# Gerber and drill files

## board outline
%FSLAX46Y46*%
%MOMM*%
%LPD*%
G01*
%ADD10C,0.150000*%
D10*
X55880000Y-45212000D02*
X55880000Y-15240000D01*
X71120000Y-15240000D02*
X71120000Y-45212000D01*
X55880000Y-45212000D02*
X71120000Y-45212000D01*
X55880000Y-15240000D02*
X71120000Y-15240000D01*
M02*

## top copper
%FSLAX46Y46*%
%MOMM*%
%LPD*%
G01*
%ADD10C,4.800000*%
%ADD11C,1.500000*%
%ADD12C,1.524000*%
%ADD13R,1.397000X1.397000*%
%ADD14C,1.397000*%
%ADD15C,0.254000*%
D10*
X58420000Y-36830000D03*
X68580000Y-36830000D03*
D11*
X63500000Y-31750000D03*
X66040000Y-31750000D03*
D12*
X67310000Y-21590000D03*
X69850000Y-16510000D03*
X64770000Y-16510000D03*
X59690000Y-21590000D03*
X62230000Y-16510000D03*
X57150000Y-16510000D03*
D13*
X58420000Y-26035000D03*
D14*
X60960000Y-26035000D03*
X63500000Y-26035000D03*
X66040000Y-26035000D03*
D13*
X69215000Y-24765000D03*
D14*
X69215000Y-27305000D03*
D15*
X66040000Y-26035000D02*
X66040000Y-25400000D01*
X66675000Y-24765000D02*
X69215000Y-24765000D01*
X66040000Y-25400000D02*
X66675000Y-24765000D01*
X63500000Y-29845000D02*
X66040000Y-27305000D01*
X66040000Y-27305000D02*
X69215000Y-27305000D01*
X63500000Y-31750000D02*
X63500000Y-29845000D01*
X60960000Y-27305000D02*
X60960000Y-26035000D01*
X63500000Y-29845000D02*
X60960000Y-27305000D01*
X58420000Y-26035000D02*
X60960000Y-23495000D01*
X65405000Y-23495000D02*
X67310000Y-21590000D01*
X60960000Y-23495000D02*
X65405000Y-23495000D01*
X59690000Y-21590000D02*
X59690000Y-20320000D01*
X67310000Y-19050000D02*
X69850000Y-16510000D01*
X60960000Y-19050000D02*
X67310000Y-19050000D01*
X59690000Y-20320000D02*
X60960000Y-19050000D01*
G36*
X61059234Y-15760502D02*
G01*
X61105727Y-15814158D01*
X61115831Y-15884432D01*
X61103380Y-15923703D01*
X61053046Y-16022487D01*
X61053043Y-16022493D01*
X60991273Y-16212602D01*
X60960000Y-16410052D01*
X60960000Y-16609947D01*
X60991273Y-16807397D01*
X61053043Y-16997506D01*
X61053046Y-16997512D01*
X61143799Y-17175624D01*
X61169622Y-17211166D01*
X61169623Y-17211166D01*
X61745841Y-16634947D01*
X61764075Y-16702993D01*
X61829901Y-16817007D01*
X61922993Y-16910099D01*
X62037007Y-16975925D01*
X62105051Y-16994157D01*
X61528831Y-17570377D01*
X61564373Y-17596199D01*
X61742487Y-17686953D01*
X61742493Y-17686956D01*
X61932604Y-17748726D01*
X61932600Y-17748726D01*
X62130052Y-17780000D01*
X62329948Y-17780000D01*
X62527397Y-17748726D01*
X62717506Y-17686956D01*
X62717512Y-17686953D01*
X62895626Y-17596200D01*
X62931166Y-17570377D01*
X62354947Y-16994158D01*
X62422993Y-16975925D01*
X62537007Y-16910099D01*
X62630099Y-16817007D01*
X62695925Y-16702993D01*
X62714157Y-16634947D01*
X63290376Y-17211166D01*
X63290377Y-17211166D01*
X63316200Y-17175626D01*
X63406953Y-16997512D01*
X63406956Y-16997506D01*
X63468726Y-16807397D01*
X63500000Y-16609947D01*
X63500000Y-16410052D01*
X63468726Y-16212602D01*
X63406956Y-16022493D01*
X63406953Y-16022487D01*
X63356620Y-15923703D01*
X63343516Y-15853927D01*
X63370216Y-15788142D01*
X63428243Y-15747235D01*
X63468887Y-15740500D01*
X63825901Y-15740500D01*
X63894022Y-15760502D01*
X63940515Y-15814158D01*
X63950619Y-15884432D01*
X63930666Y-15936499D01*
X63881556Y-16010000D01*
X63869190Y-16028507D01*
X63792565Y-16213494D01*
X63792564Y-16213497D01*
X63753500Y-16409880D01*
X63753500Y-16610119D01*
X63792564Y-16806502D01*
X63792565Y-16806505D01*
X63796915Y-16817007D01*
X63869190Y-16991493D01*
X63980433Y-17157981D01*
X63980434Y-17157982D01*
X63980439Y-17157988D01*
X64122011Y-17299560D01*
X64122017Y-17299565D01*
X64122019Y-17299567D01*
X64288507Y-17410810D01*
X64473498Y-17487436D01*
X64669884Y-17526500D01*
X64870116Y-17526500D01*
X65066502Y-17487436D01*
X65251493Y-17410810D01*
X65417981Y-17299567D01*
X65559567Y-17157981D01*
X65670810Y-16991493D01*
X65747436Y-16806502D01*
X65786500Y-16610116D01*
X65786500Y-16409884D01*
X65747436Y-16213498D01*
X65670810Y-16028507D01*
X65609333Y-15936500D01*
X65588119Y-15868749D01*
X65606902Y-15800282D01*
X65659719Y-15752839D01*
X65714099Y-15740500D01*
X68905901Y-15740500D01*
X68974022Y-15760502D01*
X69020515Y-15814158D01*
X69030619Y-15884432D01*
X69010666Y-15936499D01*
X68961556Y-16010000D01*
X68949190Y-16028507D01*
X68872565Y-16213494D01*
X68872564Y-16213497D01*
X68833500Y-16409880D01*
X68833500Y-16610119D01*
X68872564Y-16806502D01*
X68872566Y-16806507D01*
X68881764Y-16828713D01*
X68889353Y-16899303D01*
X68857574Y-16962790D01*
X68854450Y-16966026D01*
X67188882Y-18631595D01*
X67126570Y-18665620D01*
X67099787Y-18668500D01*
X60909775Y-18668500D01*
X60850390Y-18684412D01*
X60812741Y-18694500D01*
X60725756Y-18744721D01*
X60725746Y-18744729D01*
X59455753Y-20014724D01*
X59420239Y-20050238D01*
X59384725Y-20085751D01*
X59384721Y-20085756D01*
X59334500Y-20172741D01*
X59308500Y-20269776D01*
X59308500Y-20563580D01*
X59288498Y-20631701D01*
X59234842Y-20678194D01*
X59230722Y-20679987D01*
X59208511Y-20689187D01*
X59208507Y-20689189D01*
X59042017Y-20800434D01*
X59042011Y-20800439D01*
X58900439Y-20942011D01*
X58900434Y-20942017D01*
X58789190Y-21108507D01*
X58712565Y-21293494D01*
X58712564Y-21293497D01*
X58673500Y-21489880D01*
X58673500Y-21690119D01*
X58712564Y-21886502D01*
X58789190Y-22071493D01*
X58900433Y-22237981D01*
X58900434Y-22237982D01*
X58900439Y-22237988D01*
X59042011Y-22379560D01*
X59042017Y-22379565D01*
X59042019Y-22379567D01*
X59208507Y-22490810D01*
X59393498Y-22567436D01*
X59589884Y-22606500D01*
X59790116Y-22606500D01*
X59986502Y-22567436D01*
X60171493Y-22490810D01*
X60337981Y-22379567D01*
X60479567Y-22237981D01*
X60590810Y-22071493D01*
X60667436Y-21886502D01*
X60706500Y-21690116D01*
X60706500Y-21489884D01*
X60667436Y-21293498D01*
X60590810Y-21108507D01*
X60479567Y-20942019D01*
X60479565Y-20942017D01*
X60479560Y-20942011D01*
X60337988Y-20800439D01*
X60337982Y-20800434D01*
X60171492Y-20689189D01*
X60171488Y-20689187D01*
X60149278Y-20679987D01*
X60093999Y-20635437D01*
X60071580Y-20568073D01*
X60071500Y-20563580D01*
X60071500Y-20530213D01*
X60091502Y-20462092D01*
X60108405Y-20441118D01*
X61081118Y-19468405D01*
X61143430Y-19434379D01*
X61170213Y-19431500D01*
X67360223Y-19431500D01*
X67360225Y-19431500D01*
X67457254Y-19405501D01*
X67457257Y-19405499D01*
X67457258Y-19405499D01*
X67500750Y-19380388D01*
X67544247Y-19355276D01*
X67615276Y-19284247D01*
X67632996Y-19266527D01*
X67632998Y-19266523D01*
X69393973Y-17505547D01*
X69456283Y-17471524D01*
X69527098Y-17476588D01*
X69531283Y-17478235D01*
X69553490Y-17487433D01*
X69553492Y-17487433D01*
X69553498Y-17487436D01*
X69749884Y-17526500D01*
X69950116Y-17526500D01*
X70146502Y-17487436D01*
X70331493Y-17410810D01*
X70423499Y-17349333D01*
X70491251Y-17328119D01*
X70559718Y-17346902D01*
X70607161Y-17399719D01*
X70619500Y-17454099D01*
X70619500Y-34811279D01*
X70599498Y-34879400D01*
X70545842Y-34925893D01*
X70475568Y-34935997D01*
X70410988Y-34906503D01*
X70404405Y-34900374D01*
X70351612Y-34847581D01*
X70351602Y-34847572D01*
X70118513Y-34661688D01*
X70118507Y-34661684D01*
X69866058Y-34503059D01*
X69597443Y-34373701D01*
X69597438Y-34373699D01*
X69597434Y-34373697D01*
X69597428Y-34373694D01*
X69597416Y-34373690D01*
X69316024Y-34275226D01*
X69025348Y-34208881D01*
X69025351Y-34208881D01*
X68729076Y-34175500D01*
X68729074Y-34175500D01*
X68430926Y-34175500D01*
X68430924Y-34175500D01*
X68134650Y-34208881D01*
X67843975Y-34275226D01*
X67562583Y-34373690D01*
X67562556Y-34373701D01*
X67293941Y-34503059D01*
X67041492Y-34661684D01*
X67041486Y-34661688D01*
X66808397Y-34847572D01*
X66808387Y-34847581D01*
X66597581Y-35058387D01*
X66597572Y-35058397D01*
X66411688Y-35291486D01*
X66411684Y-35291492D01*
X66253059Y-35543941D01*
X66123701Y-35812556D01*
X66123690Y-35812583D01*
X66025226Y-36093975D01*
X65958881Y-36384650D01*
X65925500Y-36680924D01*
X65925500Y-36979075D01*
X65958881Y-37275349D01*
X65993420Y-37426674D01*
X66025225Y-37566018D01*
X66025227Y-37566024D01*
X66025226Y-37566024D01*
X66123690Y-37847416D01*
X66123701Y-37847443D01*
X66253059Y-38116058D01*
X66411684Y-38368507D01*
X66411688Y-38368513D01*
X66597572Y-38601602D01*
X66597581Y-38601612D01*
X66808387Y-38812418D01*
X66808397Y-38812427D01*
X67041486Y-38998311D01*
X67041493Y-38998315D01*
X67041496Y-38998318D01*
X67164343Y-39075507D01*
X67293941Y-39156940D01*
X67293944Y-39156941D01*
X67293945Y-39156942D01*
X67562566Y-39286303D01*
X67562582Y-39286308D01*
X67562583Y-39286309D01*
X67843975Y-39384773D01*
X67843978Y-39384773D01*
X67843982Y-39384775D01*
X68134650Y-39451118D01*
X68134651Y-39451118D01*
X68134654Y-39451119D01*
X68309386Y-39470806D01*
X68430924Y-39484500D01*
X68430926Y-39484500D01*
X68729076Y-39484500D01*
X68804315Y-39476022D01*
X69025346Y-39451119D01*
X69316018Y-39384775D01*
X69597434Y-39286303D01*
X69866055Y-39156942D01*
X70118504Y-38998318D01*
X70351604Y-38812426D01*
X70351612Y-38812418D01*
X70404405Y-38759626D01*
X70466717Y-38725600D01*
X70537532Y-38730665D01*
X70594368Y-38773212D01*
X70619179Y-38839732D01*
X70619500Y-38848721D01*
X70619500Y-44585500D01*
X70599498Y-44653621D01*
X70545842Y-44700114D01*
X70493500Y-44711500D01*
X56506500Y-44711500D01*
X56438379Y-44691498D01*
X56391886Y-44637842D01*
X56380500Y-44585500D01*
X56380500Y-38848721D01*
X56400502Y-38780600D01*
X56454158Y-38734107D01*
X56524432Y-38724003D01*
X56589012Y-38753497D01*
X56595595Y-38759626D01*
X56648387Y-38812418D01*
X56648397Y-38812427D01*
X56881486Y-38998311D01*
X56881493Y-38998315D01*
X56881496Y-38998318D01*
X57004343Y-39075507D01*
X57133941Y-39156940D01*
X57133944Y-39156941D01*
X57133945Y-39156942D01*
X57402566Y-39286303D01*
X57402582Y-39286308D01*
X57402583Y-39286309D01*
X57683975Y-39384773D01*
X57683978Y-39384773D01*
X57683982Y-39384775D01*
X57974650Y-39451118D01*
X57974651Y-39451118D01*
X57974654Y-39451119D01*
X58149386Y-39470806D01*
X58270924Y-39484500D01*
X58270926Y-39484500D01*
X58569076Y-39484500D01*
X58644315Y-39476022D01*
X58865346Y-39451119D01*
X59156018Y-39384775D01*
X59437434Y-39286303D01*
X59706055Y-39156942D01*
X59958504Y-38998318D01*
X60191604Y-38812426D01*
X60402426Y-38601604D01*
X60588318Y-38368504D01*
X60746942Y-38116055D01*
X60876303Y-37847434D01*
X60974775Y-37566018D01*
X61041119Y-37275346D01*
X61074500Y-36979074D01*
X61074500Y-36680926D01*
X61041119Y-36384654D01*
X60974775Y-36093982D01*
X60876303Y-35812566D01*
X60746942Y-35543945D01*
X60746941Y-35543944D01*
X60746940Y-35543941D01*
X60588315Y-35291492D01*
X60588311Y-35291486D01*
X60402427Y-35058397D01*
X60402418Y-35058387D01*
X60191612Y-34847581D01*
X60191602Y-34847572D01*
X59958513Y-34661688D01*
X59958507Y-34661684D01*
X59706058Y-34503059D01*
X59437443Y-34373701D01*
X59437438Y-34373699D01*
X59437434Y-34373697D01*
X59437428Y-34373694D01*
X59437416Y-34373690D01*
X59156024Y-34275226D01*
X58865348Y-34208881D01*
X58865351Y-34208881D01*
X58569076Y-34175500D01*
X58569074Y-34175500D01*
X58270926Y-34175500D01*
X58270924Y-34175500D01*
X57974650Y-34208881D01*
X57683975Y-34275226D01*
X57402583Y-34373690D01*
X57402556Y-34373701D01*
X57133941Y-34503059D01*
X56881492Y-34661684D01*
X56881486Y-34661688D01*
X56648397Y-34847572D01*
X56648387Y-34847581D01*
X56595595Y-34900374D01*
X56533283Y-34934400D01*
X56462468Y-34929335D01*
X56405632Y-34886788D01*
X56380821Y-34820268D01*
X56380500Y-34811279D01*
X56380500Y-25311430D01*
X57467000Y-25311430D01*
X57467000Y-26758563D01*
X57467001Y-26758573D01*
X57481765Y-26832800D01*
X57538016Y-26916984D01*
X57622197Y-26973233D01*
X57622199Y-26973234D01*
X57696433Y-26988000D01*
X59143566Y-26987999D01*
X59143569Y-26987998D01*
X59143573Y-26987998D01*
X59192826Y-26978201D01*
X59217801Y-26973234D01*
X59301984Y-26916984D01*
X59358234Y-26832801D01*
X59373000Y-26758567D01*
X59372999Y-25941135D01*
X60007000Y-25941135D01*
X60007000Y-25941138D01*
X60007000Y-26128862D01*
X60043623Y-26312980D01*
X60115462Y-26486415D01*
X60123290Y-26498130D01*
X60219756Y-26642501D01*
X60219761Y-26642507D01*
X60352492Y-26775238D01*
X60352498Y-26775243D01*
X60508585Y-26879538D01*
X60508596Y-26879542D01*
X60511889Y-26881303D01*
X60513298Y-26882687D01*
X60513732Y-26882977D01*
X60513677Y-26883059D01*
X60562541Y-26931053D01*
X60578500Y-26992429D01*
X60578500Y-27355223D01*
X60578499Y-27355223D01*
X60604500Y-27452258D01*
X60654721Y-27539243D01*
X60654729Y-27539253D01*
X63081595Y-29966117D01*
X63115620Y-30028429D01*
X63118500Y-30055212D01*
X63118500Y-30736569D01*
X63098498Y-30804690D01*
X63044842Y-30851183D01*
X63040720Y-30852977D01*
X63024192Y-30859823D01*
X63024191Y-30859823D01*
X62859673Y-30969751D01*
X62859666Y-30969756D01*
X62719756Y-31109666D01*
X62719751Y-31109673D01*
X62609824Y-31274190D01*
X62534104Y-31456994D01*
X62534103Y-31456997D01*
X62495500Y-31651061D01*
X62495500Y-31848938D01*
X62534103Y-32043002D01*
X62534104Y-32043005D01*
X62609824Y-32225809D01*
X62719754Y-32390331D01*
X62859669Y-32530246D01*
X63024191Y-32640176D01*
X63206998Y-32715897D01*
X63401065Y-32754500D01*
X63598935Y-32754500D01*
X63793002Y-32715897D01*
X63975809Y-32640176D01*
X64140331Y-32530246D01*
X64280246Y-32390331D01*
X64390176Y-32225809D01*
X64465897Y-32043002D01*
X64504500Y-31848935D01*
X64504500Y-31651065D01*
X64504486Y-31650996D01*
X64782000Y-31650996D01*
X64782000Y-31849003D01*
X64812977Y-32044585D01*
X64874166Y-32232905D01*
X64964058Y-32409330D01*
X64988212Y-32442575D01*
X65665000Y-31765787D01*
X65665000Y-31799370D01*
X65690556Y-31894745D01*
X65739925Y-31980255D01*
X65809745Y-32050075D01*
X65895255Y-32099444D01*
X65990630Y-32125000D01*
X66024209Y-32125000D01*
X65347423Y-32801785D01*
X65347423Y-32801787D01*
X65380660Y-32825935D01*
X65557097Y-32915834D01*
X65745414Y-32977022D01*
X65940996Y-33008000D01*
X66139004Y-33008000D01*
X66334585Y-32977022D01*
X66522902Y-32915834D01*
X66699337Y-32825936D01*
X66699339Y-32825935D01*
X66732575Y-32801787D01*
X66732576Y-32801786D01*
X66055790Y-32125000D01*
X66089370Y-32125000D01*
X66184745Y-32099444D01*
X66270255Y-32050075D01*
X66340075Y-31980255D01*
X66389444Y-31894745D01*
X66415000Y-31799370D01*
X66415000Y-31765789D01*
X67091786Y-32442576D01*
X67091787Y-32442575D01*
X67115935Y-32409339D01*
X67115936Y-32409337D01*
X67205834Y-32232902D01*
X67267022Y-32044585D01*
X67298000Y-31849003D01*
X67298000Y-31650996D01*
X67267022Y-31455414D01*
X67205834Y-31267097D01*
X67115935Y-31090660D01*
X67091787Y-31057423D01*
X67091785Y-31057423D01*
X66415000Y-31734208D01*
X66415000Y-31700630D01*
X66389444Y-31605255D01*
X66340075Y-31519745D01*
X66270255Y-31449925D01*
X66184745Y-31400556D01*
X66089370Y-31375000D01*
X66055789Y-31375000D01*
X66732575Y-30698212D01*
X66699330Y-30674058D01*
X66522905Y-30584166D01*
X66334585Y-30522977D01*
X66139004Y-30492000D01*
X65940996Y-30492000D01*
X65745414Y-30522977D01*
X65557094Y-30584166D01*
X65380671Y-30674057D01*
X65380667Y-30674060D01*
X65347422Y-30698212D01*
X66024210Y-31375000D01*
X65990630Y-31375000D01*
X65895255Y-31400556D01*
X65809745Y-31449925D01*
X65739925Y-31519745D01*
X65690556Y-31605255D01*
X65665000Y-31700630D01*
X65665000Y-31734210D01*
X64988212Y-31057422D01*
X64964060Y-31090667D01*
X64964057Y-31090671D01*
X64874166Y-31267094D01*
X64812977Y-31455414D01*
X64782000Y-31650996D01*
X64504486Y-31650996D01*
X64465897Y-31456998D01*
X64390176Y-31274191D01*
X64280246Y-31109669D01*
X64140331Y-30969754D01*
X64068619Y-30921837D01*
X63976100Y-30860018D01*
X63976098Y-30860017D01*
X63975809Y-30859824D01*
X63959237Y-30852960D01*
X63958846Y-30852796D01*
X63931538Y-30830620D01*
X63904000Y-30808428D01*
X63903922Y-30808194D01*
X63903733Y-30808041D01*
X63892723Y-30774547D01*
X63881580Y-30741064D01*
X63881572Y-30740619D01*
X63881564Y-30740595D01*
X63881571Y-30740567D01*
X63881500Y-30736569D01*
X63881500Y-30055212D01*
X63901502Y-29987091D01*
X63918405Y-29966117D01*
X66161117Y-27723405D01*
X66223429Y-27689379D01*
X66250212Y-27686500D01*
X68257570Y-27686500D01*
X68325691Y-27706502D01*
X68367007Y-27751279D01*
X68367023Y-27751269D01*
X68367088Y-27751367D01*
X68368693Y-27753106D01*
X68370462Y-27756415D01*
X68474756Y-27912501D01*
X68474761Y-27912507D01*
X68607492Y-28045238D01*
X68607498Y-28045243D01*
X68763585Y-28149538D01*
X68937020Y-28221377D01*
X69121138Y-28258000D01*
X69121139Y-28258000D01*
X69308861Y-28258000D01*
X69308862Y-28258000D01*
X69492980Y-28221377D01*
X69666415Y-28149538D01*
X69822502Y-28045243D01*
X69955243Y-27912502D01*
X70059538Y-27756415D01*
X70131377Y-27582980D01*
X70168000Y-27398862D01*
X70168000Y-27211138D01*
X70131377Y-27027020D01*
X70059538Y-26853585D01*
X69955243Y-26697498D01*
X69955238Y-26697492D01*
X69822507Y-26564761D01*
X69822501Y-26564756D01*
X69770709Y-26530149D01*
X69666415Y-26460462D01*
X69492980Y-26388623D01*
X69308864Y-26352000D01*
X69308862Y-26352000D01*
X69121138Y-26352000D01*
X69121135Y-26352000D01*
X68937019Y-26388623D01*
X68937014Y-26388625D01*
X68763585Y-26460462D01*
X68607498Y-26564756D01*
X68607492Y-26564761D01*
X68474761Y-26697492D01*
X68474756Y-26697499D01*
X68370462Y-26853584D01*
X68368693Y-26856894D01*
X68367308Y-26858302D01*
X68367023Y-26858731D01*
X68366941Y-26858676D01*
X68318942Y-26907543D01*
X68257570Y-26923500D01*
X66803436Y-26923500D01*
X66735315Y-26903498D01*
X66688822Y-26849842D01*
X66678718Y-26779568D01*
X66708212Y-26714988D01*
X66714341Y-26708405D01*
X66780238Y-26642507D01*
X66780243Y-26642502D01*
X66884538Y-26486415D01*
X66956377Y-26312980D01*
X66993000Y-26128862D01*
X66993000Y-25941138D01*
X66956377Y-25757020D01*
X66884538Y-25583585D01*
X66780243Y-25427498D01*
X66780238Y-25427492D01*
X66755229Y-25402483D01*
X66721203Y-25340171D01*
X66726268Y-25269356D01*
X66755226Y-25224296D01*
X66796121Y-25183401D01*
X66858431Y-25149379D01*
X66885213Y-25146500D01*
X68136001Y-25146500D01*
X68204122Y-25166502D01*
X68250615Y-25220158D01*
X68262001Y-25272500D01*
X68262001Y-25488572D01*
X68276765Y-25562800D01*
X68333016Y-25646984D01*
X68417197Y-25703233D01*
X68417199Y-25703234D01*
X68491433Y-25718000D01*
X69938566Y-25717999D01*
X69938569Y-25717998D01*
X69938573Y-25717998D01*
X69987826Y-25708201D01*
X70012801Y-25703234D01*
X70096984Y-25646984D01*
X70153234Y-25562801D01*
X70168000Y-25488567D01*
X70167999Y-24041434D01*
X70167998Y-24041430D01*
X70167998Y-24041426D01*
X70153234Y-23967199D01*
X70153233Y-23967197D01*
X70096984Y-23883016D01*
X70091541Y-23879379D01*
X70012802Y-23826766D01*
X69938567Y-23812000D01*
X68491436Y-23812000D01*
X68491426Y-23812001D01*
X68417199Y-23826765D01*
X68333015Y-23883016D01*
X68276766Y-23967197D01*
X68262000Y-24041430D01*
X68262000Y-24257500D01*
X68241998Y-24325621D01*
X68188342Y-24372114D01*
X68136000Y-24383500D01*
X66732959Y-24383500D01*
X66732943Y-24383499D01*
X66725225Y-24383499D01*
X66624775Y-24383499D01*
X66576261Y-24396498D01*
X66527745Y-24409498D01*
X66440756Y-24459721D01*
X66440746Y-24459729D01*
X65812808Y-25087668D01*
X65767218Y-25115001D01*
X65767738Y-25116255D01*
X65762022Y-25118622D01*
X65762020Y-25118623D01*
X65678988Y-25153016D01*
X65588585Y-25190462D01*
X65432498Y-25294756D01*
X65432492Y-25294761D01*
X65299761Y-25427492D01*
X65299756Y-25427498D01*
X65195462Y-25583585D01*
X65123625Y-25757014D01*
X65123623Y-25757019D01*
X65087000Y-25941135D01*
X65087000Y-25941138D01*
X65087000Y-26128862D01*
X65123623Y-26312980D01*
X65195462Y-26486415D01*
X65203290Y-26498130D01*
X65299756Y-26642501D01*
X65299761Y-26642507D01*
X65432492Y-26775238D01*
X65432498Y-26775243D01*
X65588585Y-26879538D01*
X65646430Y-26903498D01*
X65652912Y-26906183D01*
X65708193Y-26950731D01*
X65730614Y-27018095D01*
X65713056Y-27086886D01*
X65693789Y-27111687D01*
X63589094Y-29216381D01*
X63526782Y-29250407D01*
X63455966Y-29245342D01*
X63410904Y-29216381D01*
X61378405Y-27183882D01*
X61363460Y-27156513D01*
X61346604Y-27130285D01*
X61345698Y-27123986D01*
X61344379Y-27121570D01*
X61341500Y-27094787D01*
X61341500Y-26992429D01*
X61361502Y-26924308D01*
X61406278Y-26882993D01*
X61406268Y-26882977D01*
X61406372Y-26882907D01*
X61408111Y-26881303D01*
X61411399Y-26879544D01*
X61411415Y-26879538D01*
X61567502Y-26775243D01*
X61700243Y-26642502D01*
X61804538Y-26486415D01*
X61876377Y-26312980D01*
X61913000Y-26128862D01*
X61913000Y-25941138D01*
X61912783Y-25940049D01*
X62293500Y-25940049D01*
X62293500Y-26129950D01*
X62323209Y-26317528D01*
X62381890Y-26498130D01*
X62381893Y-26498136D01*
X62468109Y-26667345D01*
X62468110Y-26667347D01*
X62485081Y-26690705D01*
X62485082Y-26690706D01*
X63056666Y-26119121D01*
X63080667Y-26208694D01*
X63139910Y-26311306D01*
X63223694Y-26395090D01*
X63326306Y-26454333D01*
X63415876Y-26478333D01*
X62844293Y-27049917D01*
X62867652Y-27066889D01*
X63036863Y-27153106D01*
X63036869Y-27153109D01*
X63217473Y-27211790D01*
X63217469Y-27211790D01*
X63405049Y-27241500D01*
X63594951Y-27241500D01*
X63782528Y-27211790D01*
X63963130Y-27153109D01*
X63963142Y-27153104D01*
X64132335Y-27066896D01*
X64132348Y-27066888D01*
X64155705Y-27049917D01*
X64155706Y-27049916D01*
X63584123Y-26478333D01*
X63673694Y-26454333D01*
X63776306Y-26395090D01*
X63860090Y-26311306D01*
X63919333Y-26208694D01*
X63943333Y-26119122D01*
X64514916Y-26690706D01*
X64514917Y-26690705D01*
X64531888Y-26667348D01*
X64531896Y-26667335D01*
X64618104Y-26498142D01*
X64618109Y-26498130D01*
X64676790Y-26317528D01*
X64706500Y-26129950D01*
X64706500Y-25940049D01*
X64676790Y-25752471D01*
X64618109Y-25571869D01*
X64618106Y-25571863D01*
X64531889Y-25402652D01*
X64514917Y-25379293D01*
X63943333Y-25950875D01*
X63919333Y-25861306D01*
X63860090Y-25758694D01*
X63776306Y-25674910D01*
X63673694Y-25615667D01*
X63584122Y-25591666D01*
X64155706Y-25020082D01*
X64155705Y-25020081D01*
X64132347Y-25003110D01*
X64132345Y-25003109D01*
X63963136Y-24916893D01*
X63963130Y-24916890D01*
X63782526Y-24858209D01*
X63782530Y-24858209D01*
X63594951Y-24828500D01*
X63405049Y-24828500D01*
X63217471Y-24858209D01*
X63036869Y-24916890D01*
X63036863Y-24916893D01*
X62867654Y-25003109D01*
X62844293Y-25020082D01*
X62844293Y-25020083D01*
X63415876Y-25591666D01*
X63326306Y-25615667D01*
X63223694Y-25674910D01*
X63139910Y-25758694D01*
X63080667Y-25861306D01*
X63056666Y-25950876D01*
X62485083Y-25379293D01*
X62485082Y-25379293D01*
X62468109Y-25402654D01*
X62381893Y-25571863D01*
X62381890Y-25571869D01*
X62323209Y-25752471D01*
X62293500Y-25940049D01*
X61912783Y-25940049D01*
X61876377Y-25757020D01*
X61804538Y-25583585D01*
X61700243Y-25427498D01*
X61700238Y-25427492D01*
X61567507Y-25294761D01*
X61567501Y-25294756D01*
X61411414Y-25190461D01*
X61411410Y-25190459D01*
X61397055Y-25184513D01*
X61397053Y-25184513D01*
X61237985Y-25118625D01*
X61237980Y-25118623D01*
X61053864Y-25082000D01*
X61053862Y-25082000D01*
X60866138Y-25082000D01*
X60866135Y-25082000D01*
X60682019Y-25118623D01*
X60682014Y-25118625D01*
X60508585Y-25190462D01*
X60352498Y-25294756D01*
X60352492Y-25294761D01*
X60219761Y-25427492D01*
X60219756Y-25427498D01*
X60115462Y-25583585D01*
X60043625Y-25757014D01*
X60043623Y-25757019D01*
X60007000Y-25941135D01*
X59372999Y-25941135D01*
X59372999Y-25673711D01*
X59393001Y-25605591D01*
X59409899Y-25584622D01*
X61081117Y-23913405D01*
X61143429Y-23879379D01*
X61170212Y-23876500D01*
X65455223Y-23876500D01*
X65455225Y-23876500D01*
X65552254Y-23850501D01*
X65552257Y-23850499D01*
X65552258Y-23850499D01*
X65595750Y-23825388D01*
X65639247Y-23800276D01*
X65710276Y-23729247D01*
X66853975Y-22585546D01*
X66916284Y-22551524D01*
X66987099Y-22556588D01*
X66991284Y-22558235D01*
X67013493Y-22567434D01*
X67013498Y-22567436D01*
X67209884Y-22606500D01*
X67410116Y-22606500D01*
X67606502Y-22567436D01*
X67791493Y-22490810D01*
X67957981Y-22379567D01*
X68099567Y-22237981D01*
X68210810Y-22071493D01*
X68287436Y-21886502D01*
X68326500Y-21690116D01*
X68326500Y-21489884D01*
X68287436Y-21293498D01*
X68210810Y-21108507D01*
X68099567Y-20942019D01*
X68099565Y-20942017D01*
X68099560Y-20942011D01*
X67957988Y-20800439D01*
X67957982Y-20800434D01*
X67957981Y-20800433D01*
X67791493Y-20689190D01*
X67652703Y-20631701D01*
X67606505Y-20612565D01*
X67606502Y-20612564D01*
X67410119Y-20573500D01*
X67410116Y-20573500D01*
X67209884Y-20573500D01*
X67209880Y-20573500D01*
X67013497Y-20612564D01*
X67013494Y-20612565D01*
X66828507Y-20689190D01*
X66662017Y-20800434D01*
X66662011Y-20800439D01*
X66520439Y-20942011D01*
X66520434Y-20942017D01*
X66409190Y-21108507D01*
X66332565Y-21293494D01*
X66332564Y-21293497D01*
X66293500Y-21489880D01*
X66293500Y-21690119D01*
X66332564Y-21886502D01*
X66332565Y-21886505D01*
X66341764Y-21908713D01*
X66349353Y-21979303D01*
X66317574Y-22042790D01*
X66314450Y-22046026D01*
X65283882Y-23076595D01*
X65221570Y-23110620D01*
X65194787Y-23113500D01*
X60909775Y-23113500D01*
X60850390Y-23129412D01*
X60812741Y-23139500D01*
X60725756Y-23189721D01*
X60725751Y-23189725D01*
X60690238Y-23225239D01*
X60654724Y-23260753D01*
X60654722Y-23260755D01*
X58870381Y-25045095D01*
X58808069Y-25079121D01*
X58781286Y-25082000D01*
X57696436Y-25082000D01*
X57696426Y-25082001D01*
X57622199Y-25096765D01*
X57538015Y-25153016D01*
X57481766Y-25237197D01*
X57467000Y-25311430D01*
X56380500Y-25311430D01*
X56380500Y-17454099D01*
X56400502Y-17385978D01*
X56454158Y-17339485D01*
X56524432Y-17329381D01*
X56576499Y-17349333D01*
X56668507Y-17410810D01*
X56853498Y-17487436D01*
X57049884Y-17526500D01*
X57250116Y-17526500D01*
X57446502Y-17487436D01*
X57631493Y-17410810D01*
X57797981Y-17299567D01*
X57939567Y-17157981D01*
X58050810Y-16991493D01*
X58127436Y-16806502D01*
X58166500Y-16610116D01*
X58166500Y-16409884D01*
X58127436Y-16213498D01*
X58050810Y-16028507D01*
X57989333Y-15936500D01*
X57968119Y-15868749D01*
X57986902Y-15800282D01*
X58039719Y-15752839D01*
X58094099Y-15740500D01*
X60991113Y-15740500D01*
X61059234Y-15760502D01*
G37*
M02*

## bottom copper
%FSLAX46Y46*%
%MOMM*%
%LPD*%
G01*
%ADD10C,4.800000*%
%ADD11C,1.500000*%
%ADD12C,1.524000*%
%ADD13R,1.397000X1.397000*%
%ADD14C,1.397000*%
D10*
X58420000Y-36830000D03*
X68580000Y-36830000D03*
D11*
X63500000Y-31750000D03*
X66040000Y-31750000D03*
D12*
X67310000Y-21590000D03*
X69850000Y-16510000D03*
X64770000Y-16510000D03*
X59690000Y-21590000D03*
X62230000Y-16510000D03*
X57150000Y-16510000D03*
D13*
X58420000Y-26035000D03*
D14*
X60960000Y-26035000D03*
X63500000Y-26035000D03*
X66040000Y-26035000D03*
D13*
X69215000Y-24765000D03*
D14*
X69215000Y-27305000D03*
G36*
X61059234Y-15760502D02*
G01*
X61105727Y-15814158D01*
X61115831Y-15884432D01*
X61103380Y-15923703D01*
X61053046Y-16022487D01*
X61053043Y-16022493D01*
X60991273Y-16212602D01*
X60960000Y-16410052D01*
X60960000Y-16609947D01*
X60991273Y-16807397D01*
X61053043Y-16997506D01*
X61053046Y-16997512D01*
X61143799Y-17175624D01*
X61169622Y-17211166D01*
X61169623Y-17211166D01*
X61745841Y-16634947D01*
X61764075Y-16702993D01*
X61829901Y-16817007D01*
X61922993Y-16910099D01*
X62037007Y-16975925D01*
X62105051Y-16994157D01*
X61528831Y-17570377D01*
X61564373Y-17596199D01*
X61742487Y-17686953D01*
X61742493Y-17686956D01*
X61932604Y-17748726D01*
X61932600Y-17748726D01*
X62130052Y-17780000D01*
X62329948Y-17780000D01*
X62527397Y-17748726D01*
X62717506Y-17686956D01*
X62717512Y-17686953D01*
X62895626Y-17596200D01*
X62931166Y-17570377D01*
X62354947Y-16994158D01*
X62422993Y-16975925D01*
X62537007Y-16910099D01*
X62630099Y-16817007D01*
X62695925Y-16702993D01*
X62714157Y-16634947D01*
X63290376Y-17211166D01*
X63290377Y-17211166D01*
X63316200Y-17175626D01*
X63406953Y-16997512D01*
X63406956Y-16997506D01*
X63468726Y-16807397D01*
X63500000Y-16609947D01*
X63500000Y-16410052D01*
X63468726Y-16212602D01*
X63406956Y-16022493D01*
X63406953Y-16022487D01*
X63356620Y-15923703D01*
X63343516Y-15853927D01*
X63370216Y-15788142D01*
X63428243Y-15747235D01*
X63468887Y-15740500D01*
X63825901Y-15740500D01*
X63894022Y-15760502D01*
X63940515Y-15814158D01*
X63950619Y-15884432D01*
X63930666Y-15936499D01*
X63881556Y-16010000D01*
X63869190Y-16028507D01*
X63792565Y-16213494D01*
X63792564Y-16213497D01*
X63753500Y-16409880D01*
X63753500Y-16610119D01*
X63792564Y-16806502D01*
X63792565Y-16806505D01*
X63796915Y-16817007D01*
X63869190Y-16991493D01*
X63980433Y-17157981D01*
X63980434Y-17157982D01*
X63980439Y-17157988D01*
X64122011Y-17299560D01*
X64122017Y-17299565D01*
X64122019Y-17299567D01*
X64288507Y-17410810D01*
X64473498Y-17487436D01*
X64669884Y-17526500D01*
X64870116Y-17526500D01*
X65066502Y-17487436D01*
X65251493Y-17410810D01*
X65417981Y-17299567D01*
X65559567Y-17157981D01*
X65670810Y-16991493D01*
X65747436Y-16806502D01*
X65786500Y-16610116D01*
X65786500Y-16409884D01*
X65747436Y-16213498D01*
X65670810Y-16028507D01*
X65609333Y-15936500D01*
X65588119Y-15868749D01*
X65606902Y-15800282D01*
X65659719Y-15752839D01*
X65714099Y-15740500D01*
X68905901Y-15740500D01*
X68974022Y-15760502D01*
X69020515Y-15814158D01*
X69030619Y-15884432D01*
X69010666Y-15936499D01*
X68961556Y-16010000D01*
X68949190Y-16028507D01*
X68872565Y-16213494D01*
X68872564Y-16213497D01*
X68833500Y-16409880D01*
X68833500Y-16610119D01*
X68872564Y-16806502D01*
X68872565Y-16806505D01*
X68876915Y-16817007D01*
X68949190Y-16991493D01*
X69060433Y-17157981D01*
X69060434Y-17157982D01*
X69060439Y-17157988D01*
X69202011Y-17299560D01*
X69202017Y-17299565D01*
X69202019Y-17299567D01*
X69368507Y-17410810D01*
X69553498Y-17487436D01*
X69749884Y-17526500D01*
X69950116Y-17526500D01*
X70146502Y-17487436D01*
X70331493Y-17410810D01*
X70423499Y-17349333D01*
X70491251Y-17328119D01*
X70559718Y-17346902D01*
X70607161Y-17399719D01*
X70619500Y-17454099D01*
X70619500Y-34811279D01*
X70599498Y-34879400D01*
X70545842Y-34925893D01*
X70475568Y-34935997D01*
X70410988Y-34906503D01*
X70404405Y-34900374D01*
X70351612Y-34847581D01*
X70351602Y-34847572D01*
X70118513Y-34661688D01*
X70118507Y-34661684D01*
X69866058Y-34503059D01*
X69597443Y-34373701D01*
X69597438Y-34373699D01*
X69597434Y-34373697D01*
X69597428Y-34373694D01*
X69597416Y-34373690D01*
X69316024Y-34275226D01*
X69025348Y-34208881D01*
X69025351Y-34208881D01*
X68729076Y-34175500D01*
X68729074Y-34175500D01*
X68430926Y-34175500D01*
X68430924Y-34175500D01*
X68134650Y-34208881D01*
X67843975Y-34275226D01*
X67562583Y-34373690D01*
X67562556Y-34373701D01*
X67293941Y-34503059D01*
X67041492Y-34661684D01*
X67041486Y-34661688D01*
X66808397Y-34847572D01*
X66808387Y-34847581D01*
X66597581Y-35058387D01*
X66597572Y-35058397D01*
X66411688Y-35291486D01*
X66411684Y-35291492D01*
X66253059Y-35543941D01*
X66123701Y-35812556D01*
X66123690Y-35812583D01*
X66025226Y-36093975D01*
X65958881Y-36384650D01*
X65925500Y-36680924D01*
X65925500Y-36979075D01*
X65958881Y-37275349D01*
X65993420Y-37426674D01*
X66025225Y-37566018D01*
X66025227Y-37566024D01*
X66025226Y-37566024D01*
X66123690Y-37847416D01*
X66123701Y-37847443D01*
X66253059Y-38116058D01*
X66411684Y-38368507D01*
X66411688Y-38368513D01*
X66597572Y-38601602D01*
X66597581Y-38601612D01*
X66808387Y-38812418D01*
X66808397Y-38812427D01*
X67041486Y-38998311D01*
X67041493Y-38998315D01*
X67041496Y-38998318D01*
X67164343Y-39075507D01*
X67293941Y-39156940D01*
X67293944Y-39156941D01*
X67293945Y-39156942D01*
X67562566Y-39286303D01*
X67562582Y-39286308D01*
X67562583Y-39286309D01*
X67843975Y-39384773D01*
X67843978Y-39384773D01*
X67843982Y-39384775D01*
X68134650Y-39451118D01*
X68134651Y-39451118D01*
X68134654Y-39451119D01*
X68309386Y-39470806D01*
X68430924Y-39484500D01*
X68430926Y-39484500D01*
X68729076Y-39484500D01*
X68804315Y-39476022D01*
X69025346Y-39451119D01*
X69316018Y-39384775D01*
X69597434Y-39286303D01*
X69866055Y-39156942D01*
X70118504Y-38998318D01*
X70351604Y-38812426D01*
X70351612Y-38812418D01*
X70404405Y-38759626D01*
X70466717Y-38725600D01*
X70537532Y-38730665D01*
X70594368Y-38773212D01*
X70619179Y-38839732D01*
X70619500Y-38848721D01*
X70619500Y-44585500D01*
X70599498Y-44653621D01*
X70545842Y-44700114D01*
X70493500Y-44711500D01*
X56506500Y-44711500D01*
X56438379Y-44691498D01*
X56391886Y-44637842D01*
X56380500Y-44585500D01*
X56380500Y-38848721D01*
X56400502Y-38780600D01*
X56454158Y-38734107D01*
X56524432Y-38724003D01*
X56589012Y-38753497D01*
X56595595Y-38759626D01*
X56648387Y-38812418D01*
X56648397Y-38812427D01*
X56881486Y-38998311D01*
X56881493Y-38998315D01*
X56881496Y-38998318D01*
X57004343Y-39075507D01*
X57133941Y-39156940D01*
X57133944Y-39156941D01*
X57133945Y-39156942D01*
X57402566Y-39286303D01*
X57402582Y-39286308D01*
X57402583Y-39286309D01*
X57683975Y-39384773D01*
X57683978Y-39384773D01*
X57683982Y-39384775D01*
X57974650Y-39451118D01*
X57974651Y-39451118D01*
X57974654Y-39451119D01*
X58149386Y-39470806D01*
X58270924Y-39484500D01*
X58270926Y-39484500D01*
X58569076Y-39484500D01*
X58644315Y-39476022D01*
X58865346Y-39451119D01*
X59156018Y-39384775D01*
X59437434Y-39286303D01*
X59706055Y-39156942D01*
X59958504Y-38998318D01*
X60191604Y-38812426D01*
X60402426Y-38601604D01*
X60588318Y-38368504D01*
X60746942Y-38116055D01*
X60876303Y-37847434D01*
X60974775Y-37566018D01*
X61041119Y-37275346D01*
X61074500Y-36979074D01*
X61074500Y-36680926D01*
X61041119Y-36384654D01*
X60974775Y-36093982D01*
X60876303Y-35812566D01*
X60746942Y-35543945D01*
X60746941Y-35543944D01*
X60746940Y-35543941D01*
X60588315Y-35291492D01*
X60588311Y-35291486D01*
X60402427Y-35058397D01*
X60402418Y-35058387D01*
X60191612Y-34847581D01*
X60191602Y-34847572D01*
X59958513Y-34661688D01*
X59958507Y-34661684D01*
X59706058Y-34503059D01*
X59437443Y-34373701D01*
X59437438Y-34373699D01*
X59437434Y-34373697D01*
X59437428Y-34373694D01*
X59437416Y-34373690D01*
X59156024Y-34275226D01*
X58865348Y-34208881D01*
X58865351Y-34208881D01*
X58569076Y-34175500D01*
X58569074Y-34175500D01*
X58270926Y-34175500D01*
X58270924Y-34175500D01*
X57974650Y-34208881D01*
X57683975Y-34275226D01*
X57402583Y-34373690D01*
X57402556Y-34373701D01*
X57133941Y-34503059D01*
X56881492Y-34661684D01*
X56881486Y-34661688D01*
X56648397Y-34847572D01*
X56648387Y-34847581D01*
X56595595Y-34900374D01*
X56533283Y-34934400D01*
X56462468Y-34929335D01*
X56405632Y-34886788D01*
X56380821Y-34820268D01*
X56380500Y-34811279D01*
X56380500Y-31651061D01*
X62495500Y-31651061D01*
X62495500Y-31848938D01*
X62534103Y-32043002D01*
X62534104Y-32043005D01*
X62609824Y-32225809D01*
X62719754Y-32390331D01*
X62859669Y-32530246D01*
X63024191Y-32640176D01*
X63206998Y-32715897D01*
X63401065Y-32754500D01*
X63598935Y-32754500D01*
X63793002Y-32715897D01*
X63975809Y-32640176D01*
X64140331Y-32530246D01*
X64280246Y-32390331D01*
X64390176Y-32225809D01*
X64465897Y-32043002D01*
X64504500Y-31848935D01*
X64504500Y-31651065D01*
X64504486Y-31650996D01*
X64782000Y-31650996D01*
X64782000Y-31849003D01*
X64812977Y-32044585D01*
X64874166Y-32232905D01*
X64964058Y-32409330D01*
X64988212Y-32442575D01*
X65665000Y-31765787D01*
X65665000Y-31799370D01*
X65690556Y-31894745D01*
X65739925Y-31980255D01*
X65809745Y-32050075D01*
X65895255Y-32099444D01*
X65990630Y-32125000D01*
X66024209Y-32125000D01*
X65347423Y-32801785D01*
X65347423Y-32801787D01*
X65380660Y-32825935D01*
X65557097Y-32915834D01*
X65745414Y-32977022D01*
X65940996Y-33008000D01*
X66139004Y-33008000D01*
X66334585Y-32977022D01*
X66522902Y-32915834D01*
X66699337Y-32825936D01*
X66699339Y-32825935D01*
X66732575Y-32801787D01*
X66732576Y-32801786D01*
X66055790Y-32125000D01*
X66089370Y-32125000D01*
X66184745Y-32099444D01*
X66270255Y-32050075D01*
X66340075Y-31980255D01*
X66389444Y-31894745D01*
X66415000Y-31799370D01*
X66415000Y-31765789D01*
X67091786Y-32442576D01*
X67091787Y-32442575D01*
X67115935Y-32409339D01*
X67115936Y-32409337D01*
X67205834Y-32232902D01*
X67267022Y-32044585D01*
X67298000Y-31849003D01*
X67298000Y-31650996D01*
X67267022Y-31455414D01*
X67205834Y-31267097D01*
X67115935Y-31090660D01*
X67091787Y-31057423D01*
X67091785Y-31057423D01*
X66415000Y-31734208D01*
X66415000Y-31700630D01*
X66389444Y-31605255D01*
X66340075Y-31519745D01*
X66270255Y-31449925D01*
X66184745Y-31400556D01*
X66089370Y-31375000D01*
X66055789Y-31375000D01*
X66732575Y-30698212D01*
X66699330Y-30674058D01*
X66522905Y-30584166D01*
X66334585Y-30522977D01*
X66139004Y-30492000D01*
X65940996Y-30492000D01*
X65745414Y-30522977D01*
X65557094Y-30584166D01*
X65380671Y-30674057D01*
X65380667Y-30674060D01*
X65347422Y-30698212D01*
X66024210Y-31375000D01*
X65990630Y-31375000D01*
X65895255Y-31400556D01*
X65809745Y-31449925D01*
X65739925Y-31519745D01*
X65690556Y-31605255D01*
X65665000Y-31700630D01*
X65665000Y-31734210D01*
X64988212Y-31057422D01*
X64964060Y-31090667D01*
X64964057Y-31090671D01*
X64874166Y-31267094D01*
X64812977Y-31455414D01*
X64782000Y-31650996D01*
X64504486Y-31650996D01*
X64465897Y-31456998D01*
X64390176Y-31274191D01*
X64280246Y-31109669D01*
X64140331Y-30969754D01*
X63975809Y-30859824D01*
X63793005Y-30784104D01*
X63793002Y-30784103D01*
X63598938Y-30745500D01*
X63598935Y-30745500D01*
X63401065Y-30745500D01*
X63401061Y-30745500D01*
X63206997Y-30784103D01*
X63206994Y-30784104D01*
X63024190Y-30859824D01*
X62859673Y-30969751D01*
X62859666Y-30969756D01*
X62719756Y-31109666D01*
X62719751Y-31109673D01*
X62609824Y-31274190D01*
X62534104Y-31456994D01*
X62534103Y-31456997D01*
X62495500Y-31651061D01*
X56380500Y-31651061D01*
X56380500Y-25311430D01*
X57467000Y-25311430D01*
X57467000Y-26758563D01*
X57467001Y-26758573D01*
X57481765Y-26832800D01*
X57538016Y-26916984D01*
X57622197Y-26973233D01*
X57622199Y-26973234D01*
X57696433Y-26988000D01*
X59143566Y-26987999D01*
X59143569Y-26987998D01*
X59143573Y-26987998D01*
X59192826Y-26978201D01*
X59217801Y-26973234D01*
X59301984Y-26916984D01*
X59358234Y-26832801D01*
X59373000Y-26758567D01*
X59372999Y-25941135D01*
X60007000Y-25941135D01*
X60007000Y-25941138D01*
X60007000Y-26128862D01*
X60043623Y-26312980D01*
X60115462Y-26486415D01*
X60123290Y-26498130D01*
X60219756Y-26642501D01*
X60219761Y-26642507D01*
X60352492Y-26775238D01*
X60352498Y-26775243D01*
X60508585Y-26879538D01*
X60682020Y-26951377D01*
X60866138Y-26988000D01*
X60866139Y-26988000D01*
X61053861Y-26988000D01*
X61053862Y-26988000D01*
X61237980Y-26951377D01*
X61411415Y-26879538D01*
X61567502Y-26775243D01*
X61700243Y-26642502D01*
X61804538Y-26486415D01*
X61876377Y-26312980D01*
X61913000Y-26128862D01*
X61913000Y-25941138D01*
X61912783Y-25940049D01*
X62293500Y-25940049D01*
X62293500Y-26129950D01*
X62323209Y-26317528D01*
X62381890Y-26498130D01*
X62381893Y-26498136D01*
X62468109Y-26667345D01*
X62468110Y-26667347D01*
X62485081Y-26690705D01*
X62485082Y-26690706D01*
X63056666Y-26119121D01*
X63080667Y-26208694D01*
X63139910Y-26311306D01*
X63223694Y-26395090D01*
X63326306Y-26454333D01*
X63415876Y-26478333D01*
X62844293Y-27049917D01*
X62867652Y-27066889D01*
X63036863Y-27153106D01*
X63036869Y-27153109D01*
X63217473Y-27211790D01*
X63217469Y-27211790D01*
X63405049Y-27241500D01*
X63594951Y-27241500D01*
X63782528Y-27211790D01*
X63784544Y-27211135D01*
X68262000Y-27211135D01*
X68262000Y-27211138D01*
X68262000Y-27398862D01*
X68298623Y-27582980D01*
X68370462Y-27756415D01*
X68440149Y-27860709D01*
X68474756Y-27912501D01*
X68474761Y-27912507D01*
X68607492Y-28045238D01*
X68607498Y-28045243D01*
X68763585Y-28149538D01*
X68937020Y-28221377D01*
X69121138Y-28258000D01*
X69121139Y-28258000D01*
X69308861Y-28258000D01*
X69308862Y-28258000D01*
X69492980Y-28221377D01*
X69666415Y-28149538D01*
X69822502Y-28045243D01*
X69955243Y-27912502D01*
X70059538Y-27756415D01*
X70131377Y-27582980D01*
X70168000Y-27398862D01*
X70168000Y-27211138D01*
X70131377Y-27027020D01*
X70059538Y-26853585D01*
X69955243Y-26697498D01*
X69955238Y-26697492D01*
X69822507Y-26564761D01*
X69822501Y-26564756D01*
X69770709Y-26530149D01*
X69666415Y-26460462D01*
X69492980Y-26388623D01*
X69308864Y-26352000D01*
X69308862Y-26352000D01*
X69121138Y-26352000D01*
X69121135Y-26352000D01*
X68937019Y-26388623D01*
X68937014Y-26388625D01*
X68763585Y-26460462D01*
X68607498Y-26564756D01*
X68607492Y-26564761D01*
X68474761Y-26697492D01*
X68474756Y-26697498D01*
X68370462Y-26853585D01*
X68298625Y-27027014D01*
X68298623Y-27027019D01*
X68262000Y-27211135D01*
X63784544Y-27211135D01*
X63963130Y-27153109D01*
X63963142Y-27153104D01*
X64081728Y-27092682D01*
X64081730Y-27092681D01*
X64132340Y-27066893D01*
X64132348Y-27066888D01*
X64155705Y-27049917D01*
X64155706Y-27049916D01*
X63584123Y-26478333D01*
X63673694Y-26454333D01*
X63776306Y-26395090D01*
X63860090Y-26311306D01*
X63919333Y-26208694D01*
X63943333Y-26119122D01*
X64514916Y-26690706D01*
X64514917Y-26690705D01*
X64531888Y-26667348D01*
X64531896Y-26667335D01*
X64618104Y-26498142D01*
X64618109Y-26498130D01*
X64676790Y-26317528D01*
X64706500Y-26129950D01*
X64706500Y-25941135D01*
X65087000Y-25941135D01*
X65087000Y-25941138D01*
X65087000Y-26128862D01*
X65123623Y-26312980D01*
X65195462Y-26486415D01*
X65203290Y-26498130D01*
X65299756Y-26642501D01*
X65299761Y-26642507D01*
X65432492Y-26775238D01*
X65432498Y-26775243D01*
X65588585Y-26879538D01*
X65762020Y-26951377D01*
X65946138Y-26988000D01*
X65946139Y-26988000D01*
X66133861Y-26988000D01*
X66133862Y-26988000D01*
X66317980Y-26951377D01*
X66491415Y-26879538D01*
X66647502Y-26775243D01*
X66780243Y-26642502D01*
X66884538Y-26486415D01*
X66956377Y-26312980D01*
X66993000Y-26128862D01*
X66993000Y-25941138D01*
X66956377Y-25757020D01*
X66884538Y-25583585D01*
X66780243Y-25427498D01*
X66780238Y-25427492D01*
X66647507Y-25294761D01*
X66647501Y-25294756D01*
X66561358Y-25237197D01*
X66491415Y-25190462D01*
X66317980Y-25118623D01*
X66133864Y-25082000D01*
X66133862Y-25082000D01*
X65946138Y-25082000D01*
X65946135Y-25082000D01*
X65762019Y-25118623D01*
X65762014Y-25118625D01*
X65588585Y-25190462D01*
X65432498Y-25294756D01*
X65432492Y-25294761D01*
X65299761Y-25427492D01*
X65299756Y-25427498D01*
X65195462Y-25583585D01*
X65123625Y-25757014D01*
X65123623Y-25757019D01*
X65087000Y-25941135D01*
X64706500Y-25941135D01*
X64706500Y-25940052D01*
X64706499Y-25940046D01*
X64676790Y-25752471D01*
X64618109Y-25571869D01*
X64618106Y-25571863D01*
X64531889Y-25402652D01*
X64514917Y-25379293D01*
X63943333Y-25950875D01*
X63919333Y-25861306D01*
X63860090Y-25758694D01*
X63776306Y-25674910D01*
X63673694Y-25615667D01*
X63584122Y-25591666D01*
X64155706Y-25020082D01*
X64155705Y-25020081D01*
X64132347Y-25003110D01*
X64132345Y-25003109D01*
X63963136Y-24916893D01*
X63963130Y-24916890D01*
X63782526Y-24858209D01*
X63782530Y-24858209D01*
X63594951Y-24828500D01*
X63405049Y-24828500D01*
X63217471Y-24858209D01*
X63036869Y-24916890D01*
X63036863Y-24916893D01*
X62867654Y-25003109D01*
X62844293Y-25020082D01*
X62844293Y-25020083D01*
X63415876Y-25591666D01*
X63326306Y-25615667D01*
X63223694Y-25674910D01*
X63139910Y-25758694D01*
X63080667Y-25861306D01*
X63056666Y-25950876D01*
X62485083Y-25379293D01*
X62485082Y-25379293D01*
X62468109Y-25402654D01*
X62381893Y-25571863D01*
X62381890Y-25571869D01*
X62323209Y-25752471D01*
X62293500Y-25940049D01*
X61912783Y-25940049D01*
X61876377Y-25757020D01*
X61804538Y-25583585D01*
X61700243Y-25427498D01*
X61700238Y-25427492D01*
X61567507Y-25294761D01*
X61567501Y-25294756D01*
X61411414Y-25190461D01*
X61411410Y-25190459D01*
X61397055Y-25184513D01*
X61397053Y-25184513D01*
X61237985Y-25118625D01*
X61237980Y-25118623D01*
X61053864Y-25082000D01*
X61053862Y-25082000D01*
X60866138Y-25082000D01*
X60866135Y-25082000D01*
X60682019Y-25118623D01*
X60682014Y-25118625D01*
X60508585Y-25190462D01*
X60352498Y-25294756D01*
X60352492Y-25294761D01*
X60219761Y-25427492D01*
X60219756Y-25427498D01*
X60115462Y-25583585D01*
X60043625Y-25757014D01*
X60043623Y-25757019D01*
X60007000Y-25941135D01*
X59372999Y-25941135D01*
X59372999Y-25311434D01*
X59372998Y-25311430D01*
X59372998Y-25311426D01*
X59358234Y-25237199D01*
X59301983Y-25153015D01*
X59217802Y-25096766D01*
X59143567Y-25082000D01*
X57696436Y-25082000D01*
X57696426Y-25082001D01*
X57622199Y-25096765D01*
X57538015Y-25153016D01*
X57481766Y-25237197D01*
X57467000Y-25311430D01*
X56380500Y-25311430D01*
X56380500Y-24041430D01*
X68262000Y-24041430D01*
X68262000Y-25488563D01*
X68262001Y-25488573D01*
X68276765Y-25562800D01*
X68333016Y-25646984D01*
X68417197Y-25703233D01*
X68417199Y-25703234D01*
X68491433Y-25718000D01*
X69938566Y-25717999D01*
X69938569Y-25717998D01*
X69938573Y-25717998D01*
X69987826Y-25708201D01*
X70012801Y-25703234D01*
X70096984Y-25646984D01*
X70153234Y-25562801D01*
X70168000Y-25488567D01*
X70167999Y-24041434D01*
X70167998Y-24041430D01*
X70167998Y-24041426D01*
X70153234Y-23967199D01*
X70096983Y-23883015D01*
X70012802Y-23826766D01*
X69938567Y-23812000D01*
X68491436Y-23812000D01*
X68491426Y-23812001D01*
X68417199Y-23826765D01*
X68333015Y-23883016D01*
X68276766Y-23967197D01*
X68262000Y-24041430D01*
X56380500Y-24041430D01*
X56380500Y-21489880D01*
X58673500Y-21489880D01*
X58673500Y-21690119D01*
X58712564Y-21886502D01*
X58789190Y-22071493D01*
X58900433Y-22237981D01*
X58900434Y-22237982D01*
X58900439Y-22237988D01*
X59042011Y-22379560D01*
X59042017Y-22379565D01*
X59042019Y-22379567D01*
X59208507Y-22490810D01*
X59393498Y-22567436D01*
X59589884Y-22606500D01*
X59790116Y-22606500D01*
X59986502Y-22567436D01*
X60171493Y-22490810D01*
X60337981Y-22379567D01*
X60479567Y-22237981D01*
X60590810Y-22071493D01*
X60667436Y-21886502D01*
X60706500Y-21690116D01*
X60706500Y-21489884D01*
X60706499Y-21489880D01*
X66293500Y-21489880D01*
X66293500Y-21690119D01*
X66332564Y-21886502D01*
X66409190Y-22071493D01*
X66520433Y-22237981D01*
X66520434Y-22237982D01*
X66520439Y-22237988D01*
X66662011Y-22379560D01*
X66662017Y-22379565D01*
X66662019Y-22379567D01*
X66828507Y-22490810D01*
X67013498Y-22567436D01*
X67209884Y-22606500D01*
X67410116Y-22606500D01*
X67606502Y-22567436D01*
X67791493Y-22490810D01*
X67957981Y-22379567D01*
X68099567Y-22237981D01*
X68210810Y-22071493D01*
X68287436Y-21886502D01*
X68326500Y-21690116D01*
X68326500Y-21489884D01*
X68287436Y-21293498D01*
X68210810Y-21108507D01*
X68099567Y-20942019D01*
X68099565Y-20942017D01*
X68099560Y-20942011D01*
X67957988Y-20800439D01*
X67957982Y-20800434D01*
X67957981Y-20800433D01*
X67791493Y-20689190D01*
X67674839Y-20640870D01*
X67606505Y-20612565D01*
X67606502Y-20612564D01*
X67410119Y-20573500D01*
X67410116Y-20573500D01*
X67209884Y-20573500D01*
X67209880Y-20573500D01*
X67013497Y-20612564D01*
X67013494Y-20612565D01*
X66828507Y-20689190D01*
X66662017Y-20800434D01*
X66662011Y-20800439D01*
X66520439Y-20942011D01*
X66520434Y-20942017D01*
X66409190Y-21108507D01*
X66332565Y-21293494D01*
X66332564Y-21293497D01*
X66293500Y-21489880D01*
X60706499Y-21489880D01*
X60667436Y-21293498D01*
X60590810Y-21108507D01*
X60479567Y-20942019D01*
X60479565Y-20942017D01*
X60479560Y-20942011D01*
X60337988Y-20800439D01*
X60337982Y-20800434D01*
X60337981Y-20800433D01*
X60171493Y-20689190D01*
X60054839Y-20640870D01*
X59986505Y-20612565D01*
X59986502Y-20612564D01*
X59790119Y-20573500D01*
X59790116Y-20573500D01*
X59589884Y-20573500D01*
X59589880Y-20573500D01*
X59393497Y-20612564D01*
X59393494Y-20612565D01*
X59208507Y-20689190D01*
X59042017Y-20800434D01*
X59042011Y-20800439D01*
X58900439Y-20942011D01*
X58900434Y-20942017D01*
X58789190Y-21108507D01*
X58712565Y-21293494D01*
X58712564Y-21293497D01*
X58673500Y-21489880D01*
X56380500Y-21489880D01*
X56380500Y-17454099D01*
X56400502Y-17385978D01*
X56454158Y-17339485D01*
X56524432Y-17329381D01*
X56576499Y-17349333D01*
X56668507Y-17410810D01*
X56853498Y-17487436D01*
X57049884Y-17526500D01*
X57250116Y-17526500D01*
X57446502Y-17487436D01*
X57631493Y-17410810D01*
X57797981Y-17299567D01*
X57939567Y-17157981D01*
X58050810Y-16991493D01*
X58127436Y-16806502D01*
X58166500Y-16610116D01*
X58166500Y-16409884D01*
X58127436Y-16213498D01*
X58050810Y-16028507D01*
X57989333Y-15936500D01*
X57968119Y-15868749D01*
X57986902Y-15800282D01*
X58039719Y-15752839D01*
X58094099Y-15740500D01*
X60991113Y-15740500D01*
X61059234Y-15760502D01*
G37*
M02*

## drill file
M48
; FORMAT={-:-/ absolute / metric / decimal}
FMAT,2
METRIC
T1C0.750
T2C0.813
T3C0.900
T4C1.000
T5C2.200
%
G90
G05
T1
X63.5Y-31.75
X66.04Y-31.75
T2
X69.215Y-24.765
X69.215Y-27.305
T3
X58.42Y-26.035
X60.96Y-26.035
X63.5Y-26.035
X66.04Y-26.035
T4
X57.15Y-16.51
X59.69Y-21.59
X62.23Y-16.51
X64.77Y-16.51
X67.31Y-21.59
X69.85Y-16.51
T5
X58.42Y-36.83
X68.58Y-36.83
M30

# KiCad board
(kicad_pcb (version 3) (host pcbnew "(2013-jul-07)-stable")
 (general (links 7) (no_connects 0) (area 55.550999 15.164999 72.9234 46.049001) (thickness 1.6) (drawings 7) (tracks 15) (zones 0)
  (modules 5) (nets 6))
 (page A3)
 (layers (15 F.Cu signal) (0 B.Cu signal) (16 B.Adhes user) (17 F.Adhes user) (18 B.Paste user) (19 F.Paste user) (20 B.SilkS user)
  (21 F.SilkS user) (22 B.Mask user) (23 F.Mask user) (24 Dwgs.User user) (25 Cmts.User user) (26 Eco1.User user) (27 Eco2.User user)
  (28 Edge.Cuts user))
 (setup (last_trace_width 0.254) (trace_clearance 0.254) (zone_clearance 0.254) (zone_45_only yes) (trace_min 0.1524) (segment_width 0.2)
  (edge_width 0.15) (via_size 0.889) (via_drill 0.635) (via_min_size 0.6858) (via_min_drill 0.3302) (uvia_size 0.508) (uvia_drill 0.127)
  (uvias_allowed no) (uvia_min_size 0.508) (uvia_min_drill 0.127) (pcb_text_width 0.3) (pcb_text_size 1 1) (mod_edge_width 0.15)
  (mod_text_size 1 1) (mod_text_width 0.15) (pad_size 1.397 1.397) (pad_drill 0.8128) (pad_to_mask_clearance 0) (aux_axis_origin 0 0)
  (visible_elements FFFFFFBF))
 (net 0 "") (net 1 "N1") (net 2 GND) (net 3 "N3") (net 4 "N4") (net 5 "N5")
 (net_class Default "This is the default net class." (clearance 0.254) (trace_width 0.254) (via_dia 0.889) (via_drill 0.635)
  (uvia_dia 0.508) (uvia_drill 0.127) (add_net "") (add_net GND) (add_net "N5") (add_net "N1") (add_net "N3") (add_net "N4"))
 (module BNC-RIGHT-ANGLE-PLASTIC (layer F.Cu) (at 63.5 31.75)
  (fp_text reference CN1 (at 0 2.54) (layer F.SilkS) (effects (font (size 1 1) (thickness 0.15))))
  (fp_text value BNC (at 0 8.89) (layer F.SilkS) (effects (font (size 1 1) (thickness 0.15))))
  (pad NC thru_hole circle (at -5.08 5.08) (size 4.8 4.8) (drill 2.2) (layers *.Cu *.Mask F.SilkS))
  (pad NC thru_hole circle (at 5.08 5.08) (size 4.8 4.8) (drill 2.2) (layers *.Cu *.Mask F.SilkS))
  (pad 1 thru_hole circle (at 0 0) (size 1.5 1.5) (drill 0.75) (layers *.Cu *.Mask F.SilkS) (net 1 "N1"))
  (pad 2 thru_hole circle (at 2.54 0) (size 1.5 1.5) (drill 0.75) (layers *.Cu *.Mask F.SilkS) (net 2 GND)))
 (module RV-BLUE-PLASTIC (layer F.Cu) (at 67.31 21.59 180) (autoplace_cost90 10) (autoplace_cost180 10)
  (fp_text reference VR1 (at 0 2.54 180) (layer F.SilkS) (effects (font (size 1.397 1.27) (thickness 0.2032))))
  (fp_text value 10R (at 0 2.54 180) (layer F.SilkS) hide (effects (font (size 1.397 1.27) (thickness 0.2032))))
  (pad 2 thru_hole circle (at 0 0 180) (size 1.524 1.524) (drill 1) (layers *.Cu *.Mask F.SilkS) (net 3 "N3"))
  (pad 1 thru_hole circle (at -2.54 5.08 180) (size 1.524 1.524) (drill 1) (layers *.Cu *.Mask F.SilkS) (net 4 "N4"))
  (pad 3 thru_hole circle (at 2.54 5.08 180) (size 1.524 1.524) (drill 1) (layers *.Cu *.Mask F.SilkS)))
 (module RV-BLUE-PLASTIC (layer F.Cu) (at 59.69 21.59 180) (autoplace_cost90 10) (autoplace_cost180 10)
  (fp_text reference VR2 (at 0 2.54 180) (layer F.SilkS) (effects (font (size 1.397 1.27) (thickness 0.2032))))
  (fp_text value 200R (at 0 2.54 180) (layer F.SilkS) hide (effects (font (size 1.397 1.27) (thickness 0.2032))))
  (pad 2 thru_hole circle (at 0 0 180) (size 1.524 1.524) (drill 1) (layers *.Cu *.Mask F.SilkS) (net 4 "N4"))
  (pad 1 thru_hole circle (at -2.54 5.08 180) (size 1.524 1.524) (drill 1) (layers *.Cu *.Mask F.SilkS) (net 2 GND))
  (pad 3 thru_hole circle (at 2.54 5.08 180) (size 1.524 1.524) (drill 1) (layers *.Cu *.Mask F.SilkS)))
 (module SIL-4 (layer F.Cu) (at 62.23 26.035)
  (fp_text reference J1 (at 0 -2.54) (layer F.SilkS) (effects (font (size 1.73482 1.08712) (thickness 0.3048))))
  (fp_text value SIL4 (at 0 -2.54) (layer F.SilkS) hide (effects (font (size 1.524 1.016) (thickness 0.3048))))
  (pad 1 thru_hole rect (at -3.81 0) (size 1.397 1.397) (drill 0.9) (layers *.Cu *.Mask F.SilkS) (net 3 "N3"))
  (pad 2 thru_hole circle (at -1.27 0) (size 1.397 1.397) (drill 0.9) (layers *.Cu *.Mask F.SilkS) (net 1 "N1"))
  (pad 3 thru_hole circle (at 1.27 0) (size 1.397 1.397) (drill 0.9) (layers *.Cu *.Mask F.SilkS) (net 2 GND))
  (pad 4 thru_hole circle (at 3.81 0) (size 1.397 1.397) (drill 0.9) (layers *.Cu *.Mask F.SilkS) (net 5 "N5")))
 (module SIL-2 (layer F.Cu) (at 69.215 26.035 270)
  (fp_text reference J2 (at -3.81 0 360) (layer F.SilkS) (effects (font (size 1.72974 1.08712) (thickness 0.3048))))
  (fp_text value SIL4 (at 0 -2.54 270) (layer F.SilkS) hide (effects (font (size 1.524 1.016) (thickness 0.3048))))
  (pad 1 thru_hole rect (at -1.27 0 270) (size 1.397 1.397) (drill 0.8128) (layers *.Cu *.Mask F.SilkS) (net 5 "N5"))
  (pad 2 thru_hole circle (at 1.27 0 270) (size 1.397 1.397) (drill 0.8128) (layers *.Cu *.Mask F.SilkS) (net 1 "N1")))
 (gr_line (start 55.88 45.212) (end 55.88 15.24) (angle 90) (layer Edge.Cuts) (width 0.15))
 (gr_line (start 71.12 15.24) (end 71.12 45.212) (angle 90) (layer Edge.Cuts) (width 0.15))
 (gr_line (start 55.88 45.212) (end 71.12 45.212) (angle 90) (layer Edge.Cuts) (width 0.15))
 (gr_line (start 55.88 15.24) (end 71.12 15.24) (angle 90) (layer Edge.Cuts) (width 0.15))
 (segment (start 66.04 26.035) (end 66.04 25.4) (width 0.254) (layer F.Cu) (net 5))
 (segment (start 66.675 24.765) (end 69.215 24.765) (width 0.254) (layer F.Cu) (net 5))
 (segment (start 66.04 25.4) (end 66.675 24.765) (width 0.254) (layer F.Cu) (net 5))
 (segment (start 63.5 29.845) (end 66.04 27.305) (width 0.254) (layer F.Cu) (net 1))
 (segment (start 66.04 27.305) (end 69.215 27.305) (width 0.254) (layer F.Cu) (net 1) (status 800000))
 (segment (start 63.5 31.75) (end 63.5 29.845) (width 0.254) (layer F.Cu) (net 1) (status 10))
 (segment (start 60.96 27.305) (end 60.96 26.035) (width 0.254) (layer F.Cu) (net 1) (status 20))
 (segment (start 63.5 29.845) (end 60.96 27.305) (width 0.254) (layer F.Cu) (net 1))
 (segment (start 58.42 26.035) (end 60.96 23.495) (width 0.254) (layer F.Cu) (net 3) (status 10))
 (segment (start 65.405 23.495) (end 67.31 21.59) (width 0.254) (layer F.Cu) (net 3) (status 20))
 (segment (start 60.96 23.495) (end 65.405 23.495) (width 0.254) (layer F.Cu) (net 3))
 (segment (start 59.69 21.59) (end 59.69 20.32) (width 0.254) (layer F.Cu) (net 4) (status 10))
 (segment (start 67.31 19.05) (end 69.85 16.51) (width 0.254) (layer F.Cu) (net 4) (status 20))
 (segment (start 60.96 19.05) (end 67.31 19.05) (width 0.254) (layer F.Cu) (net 4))
 (segment (start 59.69 20.32) (end 60.96 19.05) (width 0.254) (layer F.Cu) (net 4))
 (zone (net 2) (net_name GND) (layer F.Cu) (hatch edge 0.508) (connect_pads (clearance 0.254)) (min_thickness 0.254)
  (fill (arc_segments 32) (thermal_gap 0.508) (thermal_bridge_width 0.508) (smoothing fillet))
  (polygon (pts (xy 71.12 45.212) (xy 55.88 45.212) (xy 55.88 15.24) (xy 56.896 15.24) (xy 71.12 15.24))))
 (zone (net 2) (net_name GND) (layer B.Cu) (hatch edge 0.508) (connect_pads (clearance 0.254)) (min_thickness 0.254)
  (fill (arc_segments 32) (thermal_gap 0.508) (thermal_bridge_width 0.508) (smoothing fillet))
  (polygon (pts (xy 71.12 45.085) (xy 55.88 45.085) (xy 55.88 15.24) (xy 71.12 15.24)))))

